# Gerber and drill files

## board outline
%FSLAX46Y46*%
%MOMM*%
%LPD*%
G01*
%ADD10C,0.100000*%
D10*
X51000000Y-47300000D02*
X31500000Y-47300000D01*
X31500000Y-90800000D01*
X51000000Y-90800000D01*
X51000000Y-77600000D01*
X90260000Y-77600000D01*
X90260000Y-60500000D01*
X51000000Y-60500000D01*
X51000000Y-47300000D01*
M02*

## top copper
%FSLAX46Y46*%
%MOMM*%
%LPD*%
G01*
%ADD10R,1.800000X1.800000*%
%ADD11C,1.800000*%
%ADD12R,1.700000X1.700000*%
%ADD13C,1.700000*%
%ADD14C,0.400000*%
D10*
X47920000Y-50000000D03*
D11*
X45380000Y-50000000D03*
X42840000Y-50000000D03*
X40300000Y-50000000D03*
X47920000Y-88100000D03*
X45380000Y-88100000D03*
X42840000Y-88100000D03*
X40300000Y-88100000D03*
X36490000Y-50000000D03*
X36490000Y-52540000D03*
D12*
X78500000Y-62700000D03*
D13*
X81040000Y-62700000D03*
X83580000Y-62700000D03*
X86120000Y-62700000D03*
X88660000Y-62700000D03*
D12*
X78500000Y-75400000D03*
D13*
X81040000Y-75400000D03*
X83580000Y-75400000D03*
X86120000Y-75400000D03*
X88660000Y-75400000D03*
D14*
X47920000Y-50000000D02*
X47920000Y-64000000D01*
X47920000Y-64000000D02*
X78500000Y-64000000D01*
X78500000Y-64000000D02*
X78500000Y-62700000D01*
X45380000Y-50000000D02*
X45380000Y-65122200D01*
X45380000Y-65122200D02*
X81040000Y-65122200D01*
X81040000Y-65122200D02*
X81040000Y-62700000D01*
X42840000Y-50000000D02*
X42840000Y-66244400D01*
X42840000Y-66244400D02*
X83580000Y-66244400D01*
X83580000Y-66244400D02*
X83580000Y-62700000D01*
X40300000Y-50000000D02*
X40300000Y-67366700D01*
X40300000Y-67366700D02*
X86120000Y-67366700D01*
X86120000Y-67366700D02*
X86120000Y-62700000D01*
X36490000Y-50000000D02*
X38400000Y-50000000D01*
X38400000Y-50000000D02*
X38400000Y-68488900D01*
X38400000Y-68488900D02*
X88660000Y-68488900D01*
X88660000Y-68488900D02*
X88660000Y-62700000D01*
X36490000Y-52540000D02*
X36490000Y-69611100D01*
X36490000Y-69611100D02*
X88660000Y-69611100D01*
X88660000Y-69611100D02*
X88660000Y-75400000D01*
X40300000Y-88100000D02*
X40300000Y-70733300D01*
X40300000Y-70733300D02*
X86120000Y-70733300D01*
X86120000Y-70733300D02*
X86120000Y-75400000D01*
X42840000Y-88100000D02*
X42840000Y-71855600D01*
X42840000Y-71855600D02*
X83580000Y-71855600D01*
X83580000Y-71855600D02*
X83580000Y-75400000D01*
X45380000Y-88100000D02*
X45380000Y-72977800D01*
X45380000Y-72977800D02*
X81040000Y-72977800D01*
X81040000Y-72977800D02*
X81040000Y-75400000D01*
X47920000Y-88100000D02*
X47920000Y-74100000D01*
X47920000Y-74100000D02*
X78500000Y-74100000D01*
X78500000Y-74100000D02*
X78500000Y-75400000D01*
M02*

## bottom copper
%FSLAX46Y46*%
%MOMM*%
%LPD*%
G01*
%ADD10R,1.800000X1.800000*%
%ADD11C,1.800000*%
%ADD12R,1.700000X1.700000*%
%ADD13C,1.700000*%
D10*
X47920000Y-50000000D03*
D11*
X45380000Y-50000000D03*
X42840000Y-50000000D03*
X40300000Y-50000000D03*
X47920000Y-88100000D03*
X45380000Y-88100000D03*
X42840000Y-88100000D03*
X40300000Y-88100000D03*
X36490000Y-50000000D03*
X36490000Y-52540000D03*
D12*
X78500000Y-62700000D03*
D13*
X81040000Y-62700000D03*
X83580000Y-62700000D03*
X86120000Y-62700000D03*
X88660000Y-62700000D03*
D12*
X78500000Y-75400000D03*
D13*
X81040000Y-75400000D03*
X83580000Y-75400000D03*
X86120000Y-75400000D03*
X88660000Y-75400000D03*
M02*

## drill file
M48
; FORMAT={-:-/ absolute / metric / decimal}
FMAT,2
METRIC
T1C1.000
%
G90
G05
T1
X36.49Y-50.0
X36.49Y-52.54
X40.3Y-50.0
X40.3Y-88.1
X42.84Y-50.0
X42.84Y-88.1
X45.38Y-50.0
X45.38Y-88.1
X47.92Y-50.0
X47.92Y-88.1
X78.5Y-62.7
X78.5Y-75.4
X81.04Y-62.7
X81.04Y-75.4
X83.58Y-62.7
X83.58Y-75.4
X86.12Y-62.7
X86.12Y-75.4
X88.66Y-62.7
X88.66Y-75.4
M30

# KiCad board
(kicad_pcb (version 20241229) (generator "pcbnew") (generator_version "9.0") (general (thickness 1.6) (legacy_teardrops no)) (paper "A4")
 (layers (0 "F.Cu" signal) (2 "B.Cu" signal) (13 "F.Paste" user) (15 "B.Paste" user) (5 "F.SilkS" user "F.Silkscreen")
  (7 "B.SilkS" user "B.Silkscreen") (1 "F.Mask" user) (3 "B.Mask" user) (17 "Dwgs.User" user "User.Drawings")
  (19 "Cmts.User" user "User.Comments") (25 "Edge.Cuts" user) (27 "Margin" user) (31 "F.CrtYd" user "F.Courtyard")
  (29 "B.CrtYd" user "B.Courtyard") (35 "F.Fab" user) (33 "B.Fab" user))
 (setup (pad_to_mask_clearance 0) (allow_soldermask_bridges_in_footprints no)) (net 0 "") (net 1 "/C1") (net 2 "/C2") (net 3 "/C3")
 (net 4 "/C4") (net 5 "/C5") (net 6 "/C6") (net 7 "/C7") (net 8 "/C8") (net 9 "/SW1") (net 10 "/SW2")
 (gr_poly
  (pts (xy 51.0 47.3) (xy 31.5 47.3) (xy 31.5 90.8) (xy 51.0 90.8) (xy 51.0 77.6) (xy 90.26 77.6) (xy 90.26 60.5) (xy 51.0 60.5))
  (stroke (width 0.1) (type default)) (fill no) (layer "Edge.Cuts"))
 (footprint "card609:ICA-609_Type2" (layer "B.Cu") (at 70.0 50.0)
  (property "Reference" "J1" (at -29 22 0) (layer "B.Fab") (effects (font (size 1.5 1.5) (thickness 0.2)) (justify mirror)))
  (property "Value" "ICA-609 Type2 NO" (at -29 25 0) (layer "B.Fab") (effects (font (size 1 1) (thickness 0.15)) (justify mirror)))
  (pad "C1" thru_hole rect (at -22.08 0.0) (size 1.8 1.8) (drill 1.0) (layers "F.Cu" "F.Mask") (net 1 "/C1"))
  (pad "C2" thru_hole circle (at -24.619999999999997 0.0) (size 1.8 1.8) (drill 1.0) (layers "F.Cu" "F.Mask") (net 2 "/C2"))
  (pad "C3" thru_hole circle (at -27.159999999999997 0.0) (size 1.8 1.8) (drill 1.0) (layers "F.Cu" "F.Mask") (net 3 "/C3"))
  (pad "C4" thru_hole circle (at -29.7 0.0) (size 1.8 1.8) (drill 1.0) (layers "F.Cu" "F.Mask") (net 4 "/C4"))
  (pad "C5" thru_hole circle (at -22.08 38.1) (size 1.8 1.8) (drill 1.0) (layers "F.Cu" "F.Mask") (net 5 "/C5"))
  (pad "C6" thru_hole circle (at -24.619999999999997 38.1) (size 1.8 1.8) (drill 1.0) (layers "F.Cu" "F.Mask") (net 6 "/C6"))
  (pad "C7" thru_hole circle (at -27.159999999999997 38.1) (size 1.8 1.8) (drill 1.0) (layers "F.Cu" "F.Mask") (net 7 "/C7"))
  (pad "C8" thru_hole circle (at -29.7 38.1) (size 1.8 1.8) (drill 1.0) (layers "F.Cu" "F.Mask") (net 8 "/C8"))
  (pad "SW1" thru_hole circle (at -33.51 0.0) (size 1.8 1.8) (drill 1.0) (layers "F.Cu" "F.Mask") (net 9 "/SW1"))
  (pad "SW2" thru_hole circle (at -33.51 2.54) (size 1.8 1.8) (drill 1.0) (layers "F.Cu" "F.Mask") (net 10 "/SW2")))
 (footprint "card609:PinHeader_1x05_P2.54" (layer "F.Cu") (at 78.5 62.7)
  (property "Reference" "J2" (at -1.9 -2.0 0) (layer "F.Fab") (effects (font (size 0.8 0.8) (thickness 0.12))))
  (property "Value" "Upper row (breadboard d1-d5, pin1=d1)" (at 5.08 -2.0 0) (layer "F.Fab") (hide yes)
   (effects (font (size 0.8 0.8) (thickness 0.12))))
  (pad "1" thru_hole rect (at 0.0 0) (size 1.7 1.7) (drill 1.0) (layers "F.Cu" "F.Mask") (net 1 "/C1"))
  (pad "2" thru_hole circle (at 2.54 0) (size 1.7 1.7) (drill 1.0) (layers "F.Cu" "F.Mask") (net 2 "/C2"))
  (pad "3" thru_hole circle (at 5.08 0) (size 1.7 1.7) (drill 1.0) (layers "F.Cu" "F.Mask") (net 3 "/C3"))
  (pad "4" thru_hole circle (at 7.62 0) (size 1.7 1.7) (drill 1.0) (layers "F.Cu" "F.Mask") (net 4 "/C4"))
  (pad "5" thru_hole circle (at 10.16 0) (size 1.7 1.7) (drill 1.0) (layers "F.Cu" "F.Mask") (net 9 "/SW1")))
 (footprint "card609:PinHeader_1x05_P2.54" (layer "F.Cu") (at 78.5 75.4)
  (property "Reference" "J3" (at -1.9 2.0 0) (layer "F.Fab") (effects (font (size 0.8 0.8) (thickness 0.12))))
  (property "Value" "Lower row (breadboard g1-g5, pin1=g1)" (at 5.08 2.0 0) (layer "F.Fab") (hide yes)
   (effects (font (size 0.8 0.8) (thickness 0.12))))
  (pad "1" thru_hole rect (at 0.0 0) (size 1.7 1.7) (drill 1.0) (layers "F.Cu" "F.Mask") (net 5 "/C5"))
  (pad "2" thru_hole circle (at 2.54 0) (size 1.7 1.7) (drill 1.0) (layers "F.Cu" "F.Mask") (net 6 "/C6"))
  (pad "3" thru_hole circle (at 5.08 0) (size 1.7 1.7) (drill 1.0) (layers "F.Cu" "F.Mask") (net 7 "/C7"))
  (pad "4" thru_hole circle (at 7.62 0) (size 1.7 1.7) (drill 1.0) (layers "F.Cu" "F.Mask") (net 8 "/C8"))
  (pad "5" thru_hole circle (at 10.16 0) (size 1.7 1.7) (drill 1.0) (layers "F.Cu" "F.Mask") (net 10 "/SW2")))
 (segment (start 47.92 50.0) (end 47.92 64.0) (width 0.4) (layer "F.Cu") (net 1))
 (segment (start 47.92 64.0) (end 78.5 64.0) (width 0.4) (layer "F.Cu") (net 1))
 (segment (start 78.5 64.0) (end 78.5 62.7) (width 0.4) (layer "F.Cu") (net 1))
 (segment (start 45.38 50.0) (end 45.38 65.1222) (width 0.4) (layer "F.Cu") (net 2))
 (segment (start 45.38 65.1222) (end 81.04 65.1222) (width 0.4) (layer "F.Cu") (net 2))
 (segment (start 81.04 65.1222) (end 81.04 62.7) (width 0.4) (layer "F.Cu") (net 2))
 (segment (start 42.84 50.0) (end 42.84 66.2444) (width 0.4) (layer "F.Cu") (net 3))
 (segment (start 42.84 66.2444) (end 83.58 66.2444) (width 0.4) (layer "F.Cu") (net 3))
 (segment (start 83.58 66.2444) (end 83.58 62.7) (width 0.4) (layer "F.Cu") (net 3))
 (segment (start 40.3 50.0) (end 40.3 67.3667) (width 0.4) (layer "F.Cu") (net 4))
 (segment (start 40.3 67.3667) (end 86.12 67.3667) (width 0.4) (layer "F.Cu") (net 4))
 (segment (start 86.12 67.3667) (end 86.12 62.7) (width 0.4) (layer "F.Cu") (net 4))
 (segment (start 36.49 50.0) (end 38.4 50.0) (width 0.4) (layer "F.Cu") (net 9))
 (segment (start 38.4 50.0) (end 38.4 68.4889) (width 0.4) (layer "F.Cu") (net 9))
 (segment (start 38.4 68.4889) (end 88.66 68.4889) (width 0.4) (layer "F.Cu") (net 9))
 (segment (start 88.66 68.4889) (end 88.66 62.7) (width 0.4) (layer "F.Cu") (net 9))
 (segment (start 36.49 52.54) (end 36.49 69.6111) (width 0.4) (layer "F.Cu") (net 10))
 (segment (start 36.49 69.6111) (end 88.66 69.6111) (width 0.4) (layer "F.Cu") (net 10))
 (segment (start 88.66 69.6111) (end 88.66 75.4) (width 0.4) (layer "F.Cu") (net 10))
 (segment (start 40.3 88.1) (end 40.3 70.7333) (width 0.4) (layer "F.Cu") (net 8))
 (segment (start 40.3 70.7333) (end 86.12 70.7333) (width 0.4) (layer "F.Cu") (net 8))
 (segment (start 86.12 70.7333) (end 86.12 75.4) (width 0.4) (layer "F.Cu") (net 8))
 (segment (start 42.84 88.1) (end 42.84 71.8556) (width 0.4) (layer "F.Cu") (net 7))
 (segment (start 42.84 71.8556) (end 83.58 71.8556) (width 0.4) (layer "F.Cu") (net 7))
 (segment (start 83.58 71.8556) (end 83.58 75.4) (width 0.4) (layer "F.Cu") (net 7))
 (segment (start 45.38 88.1) (end 45.38 72.9778) (width 0.4) (layer "F.Cu") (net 6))
 (segment (start 45.38 72.9778) (end 81.04 72.9778) (width 0.4) (layer "F.Cu") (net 6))
 (segment (start 81.04 72.9778) (end 81.04 75.4) (width 0.4) (layer "F.Cu") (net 6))
 (segment (start 47.92 88.1) (end 47.92 74.1) (width 0.4) (layer "F.Cu") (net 5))
 (segment (start 47.92 74.1) (end 78.5 74.1) (width 0.4) (layer "F.Cu") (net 5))
 (segment (start 78.5 74.1) (end 78.5 75.4) (width 0.4) (layer "F.Cu") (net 5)))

